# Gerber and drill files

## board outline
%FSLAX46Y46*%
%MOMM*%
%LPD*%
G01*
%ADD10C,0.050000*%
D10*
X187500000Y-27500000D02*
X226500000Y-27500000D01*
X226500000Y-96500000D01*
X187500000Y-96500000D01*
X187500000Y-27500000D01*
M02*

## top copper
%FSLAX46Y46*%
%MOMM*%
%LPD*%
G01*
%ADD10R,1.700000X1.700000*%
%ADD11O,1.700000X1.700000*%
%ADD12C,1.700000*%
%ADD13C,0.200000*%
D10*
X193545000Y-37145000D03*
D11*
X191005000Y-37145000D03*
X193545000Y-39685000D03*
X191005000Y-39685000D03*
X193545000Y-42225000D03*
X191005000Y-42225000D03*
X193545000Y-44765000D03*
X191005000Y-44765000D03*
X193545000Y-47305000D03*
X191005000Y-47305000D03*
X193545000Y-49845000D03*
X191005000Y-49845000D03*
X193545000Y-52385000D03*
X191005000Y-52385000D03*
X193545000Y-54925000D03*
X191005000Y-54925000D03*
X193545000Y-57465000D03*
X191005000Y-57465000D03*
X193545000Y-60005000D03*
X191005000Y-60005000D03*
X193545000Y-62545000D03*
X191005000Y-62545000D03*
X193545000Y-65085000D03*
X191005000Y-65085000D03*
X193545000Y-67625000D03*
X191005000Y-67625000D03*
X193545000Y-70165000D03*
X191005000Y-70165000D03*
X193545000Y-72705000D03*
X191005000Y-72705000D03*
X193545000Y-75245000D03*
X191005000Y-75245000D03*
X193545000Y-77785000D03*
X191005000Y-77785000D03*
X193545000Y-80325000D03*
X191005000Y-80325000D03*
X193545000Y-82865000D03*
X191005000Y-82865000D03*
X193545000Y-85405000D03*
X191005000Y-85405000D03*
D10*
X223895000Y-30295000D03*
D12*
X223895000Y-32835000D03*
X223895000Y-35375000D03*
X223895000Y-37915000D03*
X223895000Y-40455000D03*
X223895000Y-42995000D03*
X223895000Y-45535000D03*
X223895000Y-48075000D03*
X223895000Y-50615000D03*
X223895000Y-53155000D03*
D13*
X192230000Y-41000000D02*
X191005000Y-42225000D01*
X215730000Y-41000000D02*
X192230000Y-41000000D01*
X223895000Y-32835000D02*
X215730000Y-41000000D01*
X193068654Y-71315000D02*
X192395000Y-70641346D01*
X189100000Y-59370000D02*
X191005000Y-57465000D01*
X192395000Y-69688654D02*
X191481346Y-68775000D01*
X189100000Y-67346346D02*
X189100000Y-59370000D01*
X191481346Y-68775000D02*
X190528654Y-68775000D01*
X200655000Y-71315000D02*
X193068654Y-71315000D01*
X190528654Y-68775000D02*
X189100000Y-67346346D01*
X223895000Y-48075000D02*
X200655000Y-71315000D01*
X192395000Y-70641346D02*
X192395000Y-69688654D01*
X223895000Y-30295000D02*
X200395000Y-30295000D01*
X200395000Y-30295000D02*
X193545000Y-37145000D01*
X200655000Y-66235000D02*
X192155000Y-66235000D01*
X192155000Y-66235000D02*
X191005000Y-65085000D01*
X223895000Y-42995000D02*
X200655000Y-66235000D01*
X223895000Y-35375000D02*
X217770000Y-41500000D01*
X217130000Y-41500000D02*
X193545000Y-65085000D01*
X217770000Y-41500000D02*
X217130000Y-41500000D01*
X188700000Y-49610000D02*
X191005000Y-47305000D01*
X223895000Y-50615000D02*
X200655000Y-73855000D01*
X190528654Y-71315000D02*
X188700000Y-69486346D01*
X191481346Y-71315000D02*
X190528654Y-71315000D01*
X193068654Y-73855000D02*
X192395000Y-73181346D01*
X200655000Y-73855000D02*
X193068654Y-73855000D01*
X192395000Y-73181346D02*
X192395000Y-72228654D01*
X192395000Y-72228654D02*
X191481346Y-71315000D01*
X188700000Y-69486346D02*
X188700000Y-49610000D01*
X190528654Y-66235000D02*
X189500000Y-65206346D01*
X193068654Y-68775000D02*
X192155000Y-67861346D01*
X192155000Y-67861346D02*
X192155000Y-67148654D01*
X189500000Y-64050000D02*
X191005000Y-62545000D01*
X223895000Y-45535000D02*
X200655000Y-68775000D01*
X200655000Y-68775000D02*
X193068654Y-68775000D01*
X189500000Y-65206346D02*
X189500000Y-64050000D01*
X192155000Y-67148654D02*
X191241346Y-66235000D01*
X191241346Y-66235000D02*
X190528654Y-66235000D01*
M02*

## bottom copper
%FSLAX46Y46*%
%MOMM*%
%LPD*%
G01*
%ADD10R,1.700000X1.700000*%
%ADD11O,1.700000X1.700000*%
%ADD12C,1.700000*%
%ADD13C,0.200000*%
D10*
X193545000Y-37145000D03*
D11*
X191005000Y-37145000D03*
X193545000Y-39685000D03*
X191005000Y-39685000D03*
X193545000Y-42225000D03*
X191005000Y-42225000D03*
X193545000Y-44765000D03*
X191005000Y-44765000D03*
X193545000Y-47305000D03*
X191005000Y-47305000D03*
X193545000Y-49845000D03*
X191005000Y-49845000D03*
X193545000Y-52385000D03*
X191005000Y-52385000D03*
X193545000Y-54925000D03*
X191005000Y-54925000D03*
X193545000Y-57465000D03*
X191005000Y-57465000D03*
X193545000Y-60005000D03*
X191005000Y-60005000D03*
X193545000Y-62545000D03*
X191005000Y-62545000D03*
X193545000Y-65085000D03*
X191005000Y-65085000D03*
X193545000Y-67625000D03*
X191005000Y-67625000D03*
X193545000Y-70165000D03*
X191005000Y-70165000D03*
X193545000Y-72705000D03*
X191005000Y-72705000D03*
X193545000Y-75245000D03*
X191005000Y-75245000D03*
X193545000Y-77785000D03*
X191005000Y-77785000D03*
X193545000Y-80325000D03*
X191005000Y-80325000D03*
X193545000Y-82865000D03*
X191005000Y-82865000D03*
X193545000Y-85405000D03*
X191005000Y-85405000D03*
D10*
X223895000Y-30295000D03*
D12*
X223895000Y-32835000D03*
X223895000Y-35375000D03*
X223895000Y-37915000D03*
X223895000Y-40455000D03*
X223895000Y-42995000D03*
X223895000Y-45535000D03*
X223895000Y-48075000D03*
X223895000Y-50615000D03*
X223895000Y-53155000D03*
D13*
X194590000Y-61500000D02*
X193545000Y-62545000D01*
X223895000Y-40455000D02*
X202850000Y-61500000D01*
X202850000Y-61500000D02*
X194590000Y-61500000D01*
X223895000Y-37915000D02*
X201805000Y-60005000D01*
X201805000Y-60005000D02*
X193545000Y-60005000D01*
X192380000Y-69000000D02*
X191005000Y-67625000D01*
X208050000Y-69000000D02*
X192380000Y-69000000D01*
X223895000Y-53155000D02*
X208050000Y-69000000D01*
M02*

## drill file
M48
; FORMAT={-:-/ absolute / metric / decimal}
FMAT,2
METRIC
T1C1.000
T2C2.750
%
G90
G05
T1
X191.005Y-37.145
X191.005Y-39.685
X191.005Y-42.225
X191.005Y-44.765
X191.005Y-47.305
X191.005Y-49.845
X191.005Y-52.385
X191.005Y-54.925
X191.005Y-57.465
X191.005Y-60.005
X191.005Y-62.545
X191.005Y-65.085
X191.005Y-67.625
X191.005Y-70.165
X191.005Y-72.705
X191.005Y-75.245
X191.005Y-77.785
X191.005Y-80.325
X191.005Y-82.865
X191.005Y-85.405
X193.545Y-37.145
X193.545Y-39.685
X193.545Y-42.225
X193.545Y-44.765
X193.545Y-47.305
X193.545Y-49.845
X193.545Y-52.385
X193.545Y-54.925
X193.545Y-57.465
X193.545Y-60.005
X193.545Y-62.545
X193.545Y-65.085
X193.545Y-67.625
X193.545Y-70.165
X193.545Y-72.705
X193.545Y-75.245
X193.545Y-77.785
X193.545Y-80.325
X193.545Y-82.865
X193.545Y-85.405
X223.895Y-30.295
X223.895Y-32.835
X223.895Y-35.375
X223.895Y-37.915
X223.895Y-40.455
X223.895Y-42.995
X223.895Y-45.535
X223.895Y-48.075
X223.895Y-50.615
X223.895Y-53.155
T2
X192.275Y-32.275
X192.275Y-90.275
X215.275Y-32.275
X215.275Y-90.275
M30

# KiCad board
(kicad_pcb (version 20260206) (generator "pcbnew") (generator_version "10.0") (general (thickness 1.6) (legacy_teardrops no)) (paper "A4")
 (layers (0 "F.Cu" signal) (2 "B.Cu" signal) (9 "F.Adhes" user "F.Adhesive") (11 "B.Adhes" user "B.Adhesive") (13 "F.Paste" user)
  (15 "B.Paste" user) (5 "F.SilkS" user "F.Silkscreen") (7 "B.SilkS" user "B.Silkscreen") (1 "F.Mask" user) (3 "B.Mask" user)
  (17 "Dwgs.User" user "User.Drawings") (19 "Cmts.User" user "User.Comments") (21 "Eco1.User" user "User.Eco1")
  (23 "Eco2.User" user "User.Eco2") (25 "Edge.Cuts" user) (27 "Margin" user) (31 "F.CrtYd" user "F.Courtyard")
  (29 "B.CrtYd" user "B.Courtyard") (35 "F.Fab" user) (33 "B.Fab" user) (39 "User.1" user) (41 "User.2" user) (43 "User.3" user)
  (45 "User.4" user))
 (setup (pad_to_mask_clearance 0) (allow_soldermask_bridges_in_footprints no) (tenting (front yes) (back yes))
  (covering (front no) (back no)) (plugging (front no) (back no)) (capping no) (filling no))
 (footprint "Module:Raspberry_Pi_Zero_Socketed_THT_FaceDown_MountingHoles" (layer "F.Cu") (at 193.545 37.145)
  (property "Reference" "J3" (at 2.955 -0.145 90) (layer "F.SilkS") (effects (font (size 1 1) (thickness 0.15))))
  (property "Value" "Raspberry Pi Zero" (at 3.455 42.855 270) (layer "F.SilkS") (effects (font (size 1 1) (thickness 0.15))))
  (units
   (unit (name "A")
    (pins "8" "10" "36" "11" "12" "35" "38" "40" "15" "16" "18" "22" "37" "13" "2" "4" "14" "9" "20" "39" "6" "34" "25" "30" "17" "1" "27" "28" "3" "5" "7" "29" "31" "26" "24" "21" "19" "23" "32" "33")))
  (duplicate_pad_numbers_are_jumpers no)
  (pad "" np_thru_hole circle (at -1.27 -4.87 90) (size 2.75 2.75) (drill 2.75) (layers "*.Cu" "*.Mask") (solder_mask_margin 1.625))
  (pad "" np_thru_hole circle (at -1.27 53.13 90) (size 2.75 2.75) (drill 2.75) (layers "*.Cu" "*.Mask") (solder_mask_margin 1.625))
  (pad "" np_thru_hole circle (at 21.73 -4.87 90) (size 2.75 2.75) (drill 2.75) (layers "*.Cu" "*.Mask") (solder_mask_margin 1.625))
  (pad "" np_thru_hole circle (at 21.73 53.13 90) (size 2.75 2.75) (drill 2.75) (layers "*.Cu" "*.Mask") (solder_mask_margin 1.625))
  (pad "1" thru_hole rect (at 0 0) (size 1.7 1.7) (drill 1) (layers "*.Cu" "*.Mask") (remove_unused_layers no) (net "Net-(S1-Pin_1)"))
  (pad "2" thru_hole oval (at -2.54 0) (size 1.7 1.7) (drill 1) (layers "*.Cu" "*.Mask") (remove_unused_layers no) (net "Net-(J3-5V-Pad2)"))
  (pad "3" thru_hole oval (at 0 2.54) (size 1.7 1.7) (drill 1) (layers "*.Cu" "*.Mask") (remove_unused_layers no)
   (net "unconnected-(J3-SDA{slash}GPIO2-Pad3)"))
  (pad "4" thru_hole oval (at -2.54 2.54) (size 1.7 1.7) (drill 1) (layers "*.Cu" "*.Mask") (remove_unused_layers no)
   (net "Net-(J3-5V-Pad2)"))
  (pad "5" thru_hole oval (at 0 5.08) (size 1.7 1.7) (drill 1) (layers "*.Cu" "*.Mask") (remove_unused_layers no)
   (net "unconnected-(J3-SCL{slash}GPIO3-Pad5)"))
  (pad "6" thru_hole oval (at -2.54 5.08) (size 1.7 1.7) (drill 1) (layers "*.Cu" "*.Mask") (remove_unused_layers no) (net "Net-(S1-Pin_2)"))
  (pad "7" thru_hole oval (at 0 7.62) (size 1.7 1.7) (drill 1) (layers "*.Cu" "*.Mask") (remove_unused_layers no)
   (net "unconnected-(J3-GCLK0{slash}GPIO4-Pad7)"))
  (pad "8" thru_hole oval (at -2.54 7.62) (size 1.7 1.7) (drill 1) (layers "*.Cu" "*.Mask") (remove_unused_layers no)
   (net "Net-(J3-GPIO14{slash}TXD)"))
  (pad "9" thru_hole oval (at 0 10.16) (size 1.7 1.7) (drill 1) (layers "*.Cu" "*.Mask") (remove_unused_layers no) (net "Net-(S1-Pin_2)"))
  (pad "10" thru_hole oval (at -2.54 10.16) (size 1.7 1.7) (drill 1) (layers "*.Cu" "*.Mask") (remove_unused_layers no)
   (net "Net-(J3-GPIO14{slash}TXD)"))
  (pad "11" thru_hole oval (at 0 12.7) (size 1.7 1.7) (drill 1) (layers "*.Cu" "*.Mask") (remove_unused_layers no)
   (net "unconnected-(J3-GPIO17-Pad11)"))
  (pad "12" thru_hole oval (at -2.54 12.7) (size 1.7 1.7) (drill 1) (layers "*.Cu" "*.Mask") (remove_unused_layers no)
   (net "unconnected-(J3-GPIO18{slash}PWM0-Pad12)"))
  (pad "13" thru_hole oval (at 0 15.24) (size 1.7 1.7) (drill 1) (layers "*.Cu" "*.Mask") (remove_unused_layers no)
   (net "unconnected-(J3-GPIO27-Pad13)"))
  (pad "14" thru_hole oval (at -2.54 15.24) (size 1.7 1.7) (drill 1) (layers "*.Cu" "*.Mask") (remove_unused_layers no)
   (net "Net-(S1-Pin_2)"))
  (pad "15" thru_hole oval (at 0 17.78) (size 1.7 1.7) (drill 1) (layers "*.Cu" "*.Mask") (remove_unused_layers no)
   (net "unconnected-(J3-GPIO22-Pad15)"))
  (pad "16" thru_hole oval (at -2.54 17.78) (size 1.7 1.7) (drill 1) (layers "*.Cu" "*.Mask") (remove_unused_layers no)
   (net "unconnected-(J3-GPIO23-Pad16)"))
  (pad "17" thru_hole oval (at 0 20.32) (size 1.7 1.7) (drill 1) (layers "*.Cu" "*.Mask") (remove_unused_layers no) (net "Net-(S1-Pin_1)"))
  (pad "18" thru_hole oval (at -2.54 20.32) (size 1.7 1.7) (drill 1) (layers "*.Cu" "*.Mask") (remove_unused_layers no)
   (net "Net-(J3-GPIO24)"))
  (pad "19" thru_hole oval (at 0 22.86) (size 1.7 1.7) (drill 1) (layers "*.Cu" "*.Mask") (remove_unused_layers no)
   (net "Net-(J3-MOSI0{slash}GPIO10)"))
  (pad "20" thru_hole oval (at -2.54 22.86) (size 1.7 1.7) (drill 1) (layers "*.Cu" "*.Mask") (remove_unused_layers no)
   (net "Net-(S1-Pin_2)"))
  (pad "21" thru_hole oval (at 0 25.4) (size 1.7 1.7) (drill 1) (layers "*.Cu" "*.Mask") (remove_unused_layers no)
   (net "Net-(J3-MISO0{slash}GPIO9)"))
  (pad "22" thru_hole oval (at -2.54 25.4) (size 1.7 1.7) (drill 1) (layers "*.Cu" "*.Mask") (remove_unused_layers no)
   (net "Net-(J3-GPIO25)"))
  (pad "23" thru_hole oval (at 0 27.94) (size 1.7 1.7) (drill 1) (layers "*.Cu" "*.Mask") (remove_unused_layers no)
   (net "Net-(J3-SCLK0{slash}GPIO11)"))
  (pad "24" thru_hole oval (at -2.54 27.94) (size 1.7 1.7) (drill 1) (layers "*.Cu" "*.Mask") (remove_unused_layers no)
   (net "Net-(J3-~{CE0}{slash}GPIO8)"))
  (pad "25" thru_hole oval (at 0 30.48) (size 1.7 1.7) (drill 1) (layers "*.Cu" "*.Mask") (remove_unused_layers no) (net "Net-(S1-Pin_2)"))
  (pad "26" thru_hole oval (at -2.54 30.48) (size 1.7 1.7) (drill 1) (layers "*.Cu" "*.Mask") (remove_unused_layers no)
   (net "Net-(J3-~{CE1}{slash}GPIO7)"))
  (pad "27" thru_hole oval (at 0 33.02) (size 1.7 1.7) (drill 1) (layers "*.Cu" "*.Mask") (remove_unused_layers no)
   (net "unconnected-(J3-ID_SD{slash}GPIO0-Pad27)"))
  (pad "28" thru_hole oval (at -2.54 33.02) (size 1.7 1.7) (drill 1) (layers "*.Cu" "*.Mask") (remove_unused_layers no)
   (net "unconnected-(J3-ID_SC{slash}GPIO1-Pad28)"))
  (pad "29" thru_hole oval (at 0 35.56) (size 1.7 1.7) (drill 1) (layers "*.Cu" "*.Mask") (remove_unused_layers no)
   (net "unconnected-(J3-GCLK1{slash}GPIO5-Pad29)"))
  (pad "30" thru_hole oval (at -2.54 35.56) (size 1.7 1.7) (drill 1) (layers "*.Cu" "*.Mask") (remove_unused_layers no)
   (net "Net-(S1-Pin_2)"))
  (pad "31" thru_hole oval (at 0 38.1) (size 1.7 1.7) (drill 1) (layers "*.Cu" "*.Mask") (remove_unused_layers no)
   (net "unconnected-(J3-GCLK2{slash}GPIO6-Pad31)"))
  (pad "32" thru_hole oval (at -2.54 38.1) (size 1.7 1.7) (drill 1) (layers "*.Cu" "*.Mask") (remove_unused_layers no)
   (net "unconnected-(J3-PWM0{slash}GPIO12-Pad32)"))
  (pad "33" thru_hole oval (at 0 40.64) (size 1.7 1.7) (drill 1) (layers "*.Cu" "*.Mask") (remove_unused_layers no)
   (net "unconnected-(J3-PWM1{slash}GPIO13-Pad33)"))
  (pad "34" thru_hole oval (at -2.54 40.64) (size 1.7 1.7) (drill 1) (layers "*.Cu" "*.Mask") (remove_unused_layers no)
   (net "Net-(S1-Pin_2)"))
  (pad "35" thru_hole oval (at 0 43.18) (size 1.7 1.7) (drill 1) (layers "*.Cu" "*.Mask") (remove_unused_layers no)
   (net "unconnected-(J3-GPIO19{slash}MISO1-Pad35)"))
  (pad "36" thru_hole oval (at -2.54 43.18) (size 1.7 1.7) (drill 1) (layers "*.Cu" "*.Mask") (remove_unused_layers no)
   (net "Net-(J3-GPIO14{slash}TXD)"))
  (pad "37" thru_hole oval (at 0 45.72) (size 1.7 1.7) (drill 1) (layers "*.Cu" "*.Mask") (remove_unused_layers no)
   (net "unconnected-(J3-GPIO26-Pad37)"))
  (pad "38" thru_hole oval (at -2.54 45.72) (size 1.7 1.7) (drill 1) (layers "*.Cu" "*.Mask") (remove_unused_layers no)
   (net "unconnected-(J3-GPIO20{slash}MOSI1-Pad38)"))
  (pad "39" thru_hole oval (at 0 48.26) (size 1.7 1.7) (drill 1) (layers "*.Cu" "*.Mask") (remove_unused_layers no) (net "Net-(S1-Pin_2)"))
  (pad "40" thru_hole oval (at -2.54 48.26) (size 1.7 1.7) (drill 1) (layers "*.Cu" "*.Mask") (remove_unused_layers no)
   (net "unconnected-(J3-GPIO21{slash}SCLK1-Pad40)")))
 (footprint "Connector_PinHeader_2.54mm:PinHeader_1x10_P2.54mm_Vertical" (layer "F.Cu") (at 223.895 30.295)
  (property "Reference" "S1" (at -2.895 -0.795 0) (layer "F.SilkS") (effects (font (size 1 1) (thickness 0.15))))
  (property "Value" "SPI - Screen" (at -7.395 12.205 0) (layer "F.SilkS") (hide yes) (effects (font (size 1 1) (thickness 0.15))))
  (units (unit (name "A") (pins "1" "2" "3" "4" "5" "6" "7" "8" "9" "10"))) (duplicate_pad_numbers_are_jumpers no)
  (pad "1" thru_hole rect (at 0 0) (size 1.7 1.7) (drill 1) (layers "*.Cu" "*.Mask") (remove_unused_layers no) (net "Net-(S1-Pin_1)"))
  (pad "2" thru_hole circle (at 0 2.54) (size 1.7 1.7) (drill 1) (layers "*.Cu" "*.Mask") (remove_unused_layers no) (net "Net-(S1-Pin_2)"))
  (pad "3" thru_hole circle (at 0 5.08) (size 1.7 1.7) (drill 1) (layers "*.Cu" "*.Mask") (remove_unused_layers no)
   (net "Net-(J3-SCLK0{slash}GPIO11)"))
  (pad "4" thru_hole circle (at 0 7.62) (size 1.7 1.7) (drill 1) (layers "*.Cu" "*.Mask") (remove_unused_layers no)
   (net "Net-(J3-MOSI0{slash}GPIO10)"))
  (pad "5" thru_hole circle (at 0 10.16) (size 1.7 1.7) (drill 1) (layers "*.Cu" "*.Mask") (remove_unused_layers no)
   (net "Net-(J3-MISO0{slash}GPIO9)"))
  (pad "6" thru_hole circle (at 0 12.7) (size 1.7 1.7) (drill 1) (layers "*.Cu" "*.Mask") (remove_unused_layers no)
   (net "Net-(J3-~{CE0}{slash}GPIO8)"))
  (pad "7" thru_hole circle (at 0 15.24) (size 1.7 1.7) (drill 1) (layers "*.Cu" "*.Mask") (remove_unused_layers no) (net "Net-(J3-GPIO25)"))
  (pad "8" thru_hole circle (at 0 17.78) (size 1.7 1.7) (drill 1) (layers "*.Cu" "*.Mask") (remove_unused_layers no) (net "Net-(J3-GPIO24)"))
  (pad "9" thru_hole circle (at 0 20.32) (size 1.7 1.7) (drill 1) (layers "*.Cu" "*.Mask") (remove_unused_layers no)
   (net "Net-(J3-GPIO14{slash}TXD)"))
  (pad "10" thru_hole circle (at 0 22.86) (size 1.7 1.7) (drill 1) (layers "*.Cu" "*.Mask") (remove_unused_layers no)
   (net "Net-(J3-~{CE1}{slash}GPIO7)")))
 (gr_rect (start 187.5 27.5) (end 226.5 96.5) (stroke (width 0.05) (type default)) (fill no) (layer "Edge.Cuts"))
 (segment (start 192.23 41) (end 191.005 42.225) (width 0.2) (layer "F.Cu") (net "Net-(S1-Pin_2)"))
 (segment (start 215.73 41) (end 192.23 41) (width 0.2) (layer "F.Cu") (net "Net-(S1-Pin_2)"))
 (segment (start 223.895 32.835) (end 215.73 41) (width 0.2) (layer "F.Cu") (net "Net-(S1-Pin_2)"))
 (segment (start 194.59 61.5) (end 193.545 62.545) (width 0.2) (layer "B.Cu") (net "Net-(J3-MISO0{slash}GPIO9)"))
 (segment (start 223.895 40.455) (end 202.85 61.5) (width 0.2) (layer "B.Cu") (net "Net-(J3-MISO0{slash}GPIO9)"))
 (segment (start 202.85 61.5) (end 194.59 61.5) (width 0.2) (layer "B.Cu") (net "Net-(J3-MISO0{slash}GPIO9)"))
 (segment (start 193.068654 71.315) (end 192.395 70.641346) (width 0.2) (layer "F.Cu") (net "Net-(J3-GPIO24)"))
 (segment (start 189.1 59.37) (end 191.005 57.465) (width 0.2) (layer "F.Cu") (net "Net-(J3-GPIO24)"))
 (segment (start 192.395 69.688654) (end 191.481346 68.775) (width 0.2) (layer "F.Cu") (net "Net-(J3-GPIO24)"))
 (segment (start 189.1 67.346346) (end 189.1 59.37) (width 0.2) (layer "F.Cu") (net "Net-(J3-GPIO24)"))
 (segment (start 191.481346 68.775) (end 190.528654 68.775) (width 0.2) (layer "F.Cu") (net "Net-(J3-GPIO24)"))
 (segment (start 200.655 71.315) (end 193.068654 71.315) (width 0.2) (layer "F.Cu") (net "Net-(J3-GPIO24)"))
 (segment (start 190.528654 68.775) (end 189.1 67.346346) (width 0.2) (layer "F.Cu") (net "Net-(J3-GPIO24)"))
 (segment (start 223.895 48.075) (end 200.655 71.315) (width 0.2) (layer "F.Cu") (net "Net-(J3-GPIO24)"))
 (segment (start 192.395 70.641346) (end 192.395 69.688654) (width 0.2) (layer "F.Cu") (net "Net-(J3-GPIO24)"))
 (segment (start 223.895 30.295) (end 200.395 30.295) (width 0.2) (layer "F.Cu") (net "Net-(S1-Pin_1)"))
 (segment (start 200.395 30.295) (end 193.545 37.145) (width 0.2) (layer "F.Cu") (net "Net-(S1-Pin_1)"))
 (segment (start 200.655 66.235) (end 192.155 66.235) (width 0.2) (layer "F.Cu") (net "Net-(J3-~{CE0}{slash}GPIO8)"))
 (segment (start 192.155 66.235) (end 191.005 65.085) (width 0.2) (layer "F.Cu") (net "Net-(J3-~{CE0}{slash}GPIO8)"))
 (segment (start 223.895 42.995) (end 200.655 66.235) (width 0.2) (layer "F.Cu") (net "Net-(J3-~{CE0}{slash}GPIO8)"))
 (segment (start 223.895 35.375) (end 217.77 41.5) (width 0.2) (layer "F.Cu") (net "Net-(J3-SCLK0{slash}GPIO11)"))
 (segment (start 217.13 41.5) (end 193.545 65.085) (width 0.2) (layer "F.Cu") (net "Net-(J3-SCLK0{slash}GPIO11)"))
 (segment (start 217.77 41.5) (end 217.13 41.5) (width 0.2) (layer "F.Cu") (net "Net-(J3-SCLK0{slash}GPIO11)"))
 (segment (start 223.895 37.915) (end 201.805 60.005) (width 0.2) (layer "B.Cu") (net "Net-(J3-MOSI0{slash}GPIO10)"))
 (segment (start 201.805 60.005) (end 193.545 60.005) (width 0.2) (layer "B.Cu") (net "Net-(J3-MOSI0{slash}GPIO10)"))
 (segment (start 188.7 49.61) (end 191.005 47.305) (width 0.2) (layer "F.Cu") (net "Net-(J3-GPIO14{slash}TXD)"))
 (segment (start 223.895 50.615) (end 200.655 73.855) (width 0.2) (layer "F.Cu") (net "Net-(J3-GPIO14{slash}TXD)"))
 (segment (start 190.528654 71.315) (end 188.7 69.486346) (width 0.2) (layer "F.Cu") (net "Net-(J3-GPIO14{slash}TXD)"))
 (segment (start 191.481346 71.315) (end 190.528654 71.315) (width 0.2) (layer "F.Cu") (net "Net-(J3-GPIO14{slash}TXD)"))
 (segment (start 193.068654 73.855) (end 192.395 73.181346) (width 0.2) (layer "F.Cu") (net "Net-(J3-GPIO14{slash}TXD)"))
 (segment (start 200.655 73.855) (end 193.068654 73.855) (width 0.2) (layer "F.Cu") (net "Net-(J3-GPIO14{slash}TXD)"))
 (segment (start 192.395 73.181346) (end 192.395 72.228654) (width 0.2) (layer "F.Cu") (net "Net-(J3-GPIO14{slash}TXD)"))
 (segment (start 192.395 72.228654) (end 191.481346 71.315) (width 0.2) (layer "F.Cu") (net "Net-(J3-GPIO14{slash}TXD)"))
 (segment (start 188.7 69.486346) (end 188.7 49.61) (width 0.2) (layer "F.Cu") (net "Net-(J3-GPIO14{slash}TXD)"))
 (segment (start 192.38 69) (end 191.005 67.625) (width 0.2) (layer "B.Cu") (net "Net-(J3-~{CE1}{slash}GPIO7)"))
 (segment (start 208.05 69) (end 192.38 69) (width 0.2) (layer "B.Cu") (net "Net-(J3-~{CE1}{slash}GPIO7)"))
 (segment (start 223.895 53.155) (end 208.05 69) (width 0.2) (layer "B.Cu") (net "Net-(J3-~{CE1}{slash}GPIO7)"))
 (segment (start 190.528654 66.235) (end 189.5 65.206346) (width 0.2) (layer "F.Cu") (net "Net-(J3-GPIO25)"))
 (segment (start 193.068654 68.775) (end 192.155 67.861346) (width 0.2) (layer "F.Cu") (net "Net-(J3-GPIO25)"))
 (segment (start 192.155 67.861346) (end 192.155 67.148654) (width 0.2) (layer "F.Cu") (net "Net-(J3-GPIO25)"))
 (segment (start 189.5 64.05) (end 191.005 62.545) (width 0.2) (layer "F.Cu") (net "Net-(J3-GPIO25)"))
 (segment (start 223.895 45.535) (end 200.655 68.775) (width 0.2) (layer "F.Cu") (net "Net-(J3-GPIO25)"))
 (segment (start 200.655 68.775) (end 193.068654 68.775) (width 0.2) (layer "F.Cu") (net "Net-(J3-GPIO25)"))
 (segment (start 189.5 65.206346) (end 189.5 64.05) (width 0.2) (layer "F.Cu") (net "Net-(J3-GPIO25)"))
 (segment (start 192.155 67.148654) (end 191.241346 66.235) (width 0.2) (layer "F.Cu") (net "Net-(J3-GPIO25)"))
 (segment (start 191.241346 66.235) (end 190.528654 66.235) (width 0.2) (layer "F.Cu") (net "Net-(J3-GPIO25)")))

